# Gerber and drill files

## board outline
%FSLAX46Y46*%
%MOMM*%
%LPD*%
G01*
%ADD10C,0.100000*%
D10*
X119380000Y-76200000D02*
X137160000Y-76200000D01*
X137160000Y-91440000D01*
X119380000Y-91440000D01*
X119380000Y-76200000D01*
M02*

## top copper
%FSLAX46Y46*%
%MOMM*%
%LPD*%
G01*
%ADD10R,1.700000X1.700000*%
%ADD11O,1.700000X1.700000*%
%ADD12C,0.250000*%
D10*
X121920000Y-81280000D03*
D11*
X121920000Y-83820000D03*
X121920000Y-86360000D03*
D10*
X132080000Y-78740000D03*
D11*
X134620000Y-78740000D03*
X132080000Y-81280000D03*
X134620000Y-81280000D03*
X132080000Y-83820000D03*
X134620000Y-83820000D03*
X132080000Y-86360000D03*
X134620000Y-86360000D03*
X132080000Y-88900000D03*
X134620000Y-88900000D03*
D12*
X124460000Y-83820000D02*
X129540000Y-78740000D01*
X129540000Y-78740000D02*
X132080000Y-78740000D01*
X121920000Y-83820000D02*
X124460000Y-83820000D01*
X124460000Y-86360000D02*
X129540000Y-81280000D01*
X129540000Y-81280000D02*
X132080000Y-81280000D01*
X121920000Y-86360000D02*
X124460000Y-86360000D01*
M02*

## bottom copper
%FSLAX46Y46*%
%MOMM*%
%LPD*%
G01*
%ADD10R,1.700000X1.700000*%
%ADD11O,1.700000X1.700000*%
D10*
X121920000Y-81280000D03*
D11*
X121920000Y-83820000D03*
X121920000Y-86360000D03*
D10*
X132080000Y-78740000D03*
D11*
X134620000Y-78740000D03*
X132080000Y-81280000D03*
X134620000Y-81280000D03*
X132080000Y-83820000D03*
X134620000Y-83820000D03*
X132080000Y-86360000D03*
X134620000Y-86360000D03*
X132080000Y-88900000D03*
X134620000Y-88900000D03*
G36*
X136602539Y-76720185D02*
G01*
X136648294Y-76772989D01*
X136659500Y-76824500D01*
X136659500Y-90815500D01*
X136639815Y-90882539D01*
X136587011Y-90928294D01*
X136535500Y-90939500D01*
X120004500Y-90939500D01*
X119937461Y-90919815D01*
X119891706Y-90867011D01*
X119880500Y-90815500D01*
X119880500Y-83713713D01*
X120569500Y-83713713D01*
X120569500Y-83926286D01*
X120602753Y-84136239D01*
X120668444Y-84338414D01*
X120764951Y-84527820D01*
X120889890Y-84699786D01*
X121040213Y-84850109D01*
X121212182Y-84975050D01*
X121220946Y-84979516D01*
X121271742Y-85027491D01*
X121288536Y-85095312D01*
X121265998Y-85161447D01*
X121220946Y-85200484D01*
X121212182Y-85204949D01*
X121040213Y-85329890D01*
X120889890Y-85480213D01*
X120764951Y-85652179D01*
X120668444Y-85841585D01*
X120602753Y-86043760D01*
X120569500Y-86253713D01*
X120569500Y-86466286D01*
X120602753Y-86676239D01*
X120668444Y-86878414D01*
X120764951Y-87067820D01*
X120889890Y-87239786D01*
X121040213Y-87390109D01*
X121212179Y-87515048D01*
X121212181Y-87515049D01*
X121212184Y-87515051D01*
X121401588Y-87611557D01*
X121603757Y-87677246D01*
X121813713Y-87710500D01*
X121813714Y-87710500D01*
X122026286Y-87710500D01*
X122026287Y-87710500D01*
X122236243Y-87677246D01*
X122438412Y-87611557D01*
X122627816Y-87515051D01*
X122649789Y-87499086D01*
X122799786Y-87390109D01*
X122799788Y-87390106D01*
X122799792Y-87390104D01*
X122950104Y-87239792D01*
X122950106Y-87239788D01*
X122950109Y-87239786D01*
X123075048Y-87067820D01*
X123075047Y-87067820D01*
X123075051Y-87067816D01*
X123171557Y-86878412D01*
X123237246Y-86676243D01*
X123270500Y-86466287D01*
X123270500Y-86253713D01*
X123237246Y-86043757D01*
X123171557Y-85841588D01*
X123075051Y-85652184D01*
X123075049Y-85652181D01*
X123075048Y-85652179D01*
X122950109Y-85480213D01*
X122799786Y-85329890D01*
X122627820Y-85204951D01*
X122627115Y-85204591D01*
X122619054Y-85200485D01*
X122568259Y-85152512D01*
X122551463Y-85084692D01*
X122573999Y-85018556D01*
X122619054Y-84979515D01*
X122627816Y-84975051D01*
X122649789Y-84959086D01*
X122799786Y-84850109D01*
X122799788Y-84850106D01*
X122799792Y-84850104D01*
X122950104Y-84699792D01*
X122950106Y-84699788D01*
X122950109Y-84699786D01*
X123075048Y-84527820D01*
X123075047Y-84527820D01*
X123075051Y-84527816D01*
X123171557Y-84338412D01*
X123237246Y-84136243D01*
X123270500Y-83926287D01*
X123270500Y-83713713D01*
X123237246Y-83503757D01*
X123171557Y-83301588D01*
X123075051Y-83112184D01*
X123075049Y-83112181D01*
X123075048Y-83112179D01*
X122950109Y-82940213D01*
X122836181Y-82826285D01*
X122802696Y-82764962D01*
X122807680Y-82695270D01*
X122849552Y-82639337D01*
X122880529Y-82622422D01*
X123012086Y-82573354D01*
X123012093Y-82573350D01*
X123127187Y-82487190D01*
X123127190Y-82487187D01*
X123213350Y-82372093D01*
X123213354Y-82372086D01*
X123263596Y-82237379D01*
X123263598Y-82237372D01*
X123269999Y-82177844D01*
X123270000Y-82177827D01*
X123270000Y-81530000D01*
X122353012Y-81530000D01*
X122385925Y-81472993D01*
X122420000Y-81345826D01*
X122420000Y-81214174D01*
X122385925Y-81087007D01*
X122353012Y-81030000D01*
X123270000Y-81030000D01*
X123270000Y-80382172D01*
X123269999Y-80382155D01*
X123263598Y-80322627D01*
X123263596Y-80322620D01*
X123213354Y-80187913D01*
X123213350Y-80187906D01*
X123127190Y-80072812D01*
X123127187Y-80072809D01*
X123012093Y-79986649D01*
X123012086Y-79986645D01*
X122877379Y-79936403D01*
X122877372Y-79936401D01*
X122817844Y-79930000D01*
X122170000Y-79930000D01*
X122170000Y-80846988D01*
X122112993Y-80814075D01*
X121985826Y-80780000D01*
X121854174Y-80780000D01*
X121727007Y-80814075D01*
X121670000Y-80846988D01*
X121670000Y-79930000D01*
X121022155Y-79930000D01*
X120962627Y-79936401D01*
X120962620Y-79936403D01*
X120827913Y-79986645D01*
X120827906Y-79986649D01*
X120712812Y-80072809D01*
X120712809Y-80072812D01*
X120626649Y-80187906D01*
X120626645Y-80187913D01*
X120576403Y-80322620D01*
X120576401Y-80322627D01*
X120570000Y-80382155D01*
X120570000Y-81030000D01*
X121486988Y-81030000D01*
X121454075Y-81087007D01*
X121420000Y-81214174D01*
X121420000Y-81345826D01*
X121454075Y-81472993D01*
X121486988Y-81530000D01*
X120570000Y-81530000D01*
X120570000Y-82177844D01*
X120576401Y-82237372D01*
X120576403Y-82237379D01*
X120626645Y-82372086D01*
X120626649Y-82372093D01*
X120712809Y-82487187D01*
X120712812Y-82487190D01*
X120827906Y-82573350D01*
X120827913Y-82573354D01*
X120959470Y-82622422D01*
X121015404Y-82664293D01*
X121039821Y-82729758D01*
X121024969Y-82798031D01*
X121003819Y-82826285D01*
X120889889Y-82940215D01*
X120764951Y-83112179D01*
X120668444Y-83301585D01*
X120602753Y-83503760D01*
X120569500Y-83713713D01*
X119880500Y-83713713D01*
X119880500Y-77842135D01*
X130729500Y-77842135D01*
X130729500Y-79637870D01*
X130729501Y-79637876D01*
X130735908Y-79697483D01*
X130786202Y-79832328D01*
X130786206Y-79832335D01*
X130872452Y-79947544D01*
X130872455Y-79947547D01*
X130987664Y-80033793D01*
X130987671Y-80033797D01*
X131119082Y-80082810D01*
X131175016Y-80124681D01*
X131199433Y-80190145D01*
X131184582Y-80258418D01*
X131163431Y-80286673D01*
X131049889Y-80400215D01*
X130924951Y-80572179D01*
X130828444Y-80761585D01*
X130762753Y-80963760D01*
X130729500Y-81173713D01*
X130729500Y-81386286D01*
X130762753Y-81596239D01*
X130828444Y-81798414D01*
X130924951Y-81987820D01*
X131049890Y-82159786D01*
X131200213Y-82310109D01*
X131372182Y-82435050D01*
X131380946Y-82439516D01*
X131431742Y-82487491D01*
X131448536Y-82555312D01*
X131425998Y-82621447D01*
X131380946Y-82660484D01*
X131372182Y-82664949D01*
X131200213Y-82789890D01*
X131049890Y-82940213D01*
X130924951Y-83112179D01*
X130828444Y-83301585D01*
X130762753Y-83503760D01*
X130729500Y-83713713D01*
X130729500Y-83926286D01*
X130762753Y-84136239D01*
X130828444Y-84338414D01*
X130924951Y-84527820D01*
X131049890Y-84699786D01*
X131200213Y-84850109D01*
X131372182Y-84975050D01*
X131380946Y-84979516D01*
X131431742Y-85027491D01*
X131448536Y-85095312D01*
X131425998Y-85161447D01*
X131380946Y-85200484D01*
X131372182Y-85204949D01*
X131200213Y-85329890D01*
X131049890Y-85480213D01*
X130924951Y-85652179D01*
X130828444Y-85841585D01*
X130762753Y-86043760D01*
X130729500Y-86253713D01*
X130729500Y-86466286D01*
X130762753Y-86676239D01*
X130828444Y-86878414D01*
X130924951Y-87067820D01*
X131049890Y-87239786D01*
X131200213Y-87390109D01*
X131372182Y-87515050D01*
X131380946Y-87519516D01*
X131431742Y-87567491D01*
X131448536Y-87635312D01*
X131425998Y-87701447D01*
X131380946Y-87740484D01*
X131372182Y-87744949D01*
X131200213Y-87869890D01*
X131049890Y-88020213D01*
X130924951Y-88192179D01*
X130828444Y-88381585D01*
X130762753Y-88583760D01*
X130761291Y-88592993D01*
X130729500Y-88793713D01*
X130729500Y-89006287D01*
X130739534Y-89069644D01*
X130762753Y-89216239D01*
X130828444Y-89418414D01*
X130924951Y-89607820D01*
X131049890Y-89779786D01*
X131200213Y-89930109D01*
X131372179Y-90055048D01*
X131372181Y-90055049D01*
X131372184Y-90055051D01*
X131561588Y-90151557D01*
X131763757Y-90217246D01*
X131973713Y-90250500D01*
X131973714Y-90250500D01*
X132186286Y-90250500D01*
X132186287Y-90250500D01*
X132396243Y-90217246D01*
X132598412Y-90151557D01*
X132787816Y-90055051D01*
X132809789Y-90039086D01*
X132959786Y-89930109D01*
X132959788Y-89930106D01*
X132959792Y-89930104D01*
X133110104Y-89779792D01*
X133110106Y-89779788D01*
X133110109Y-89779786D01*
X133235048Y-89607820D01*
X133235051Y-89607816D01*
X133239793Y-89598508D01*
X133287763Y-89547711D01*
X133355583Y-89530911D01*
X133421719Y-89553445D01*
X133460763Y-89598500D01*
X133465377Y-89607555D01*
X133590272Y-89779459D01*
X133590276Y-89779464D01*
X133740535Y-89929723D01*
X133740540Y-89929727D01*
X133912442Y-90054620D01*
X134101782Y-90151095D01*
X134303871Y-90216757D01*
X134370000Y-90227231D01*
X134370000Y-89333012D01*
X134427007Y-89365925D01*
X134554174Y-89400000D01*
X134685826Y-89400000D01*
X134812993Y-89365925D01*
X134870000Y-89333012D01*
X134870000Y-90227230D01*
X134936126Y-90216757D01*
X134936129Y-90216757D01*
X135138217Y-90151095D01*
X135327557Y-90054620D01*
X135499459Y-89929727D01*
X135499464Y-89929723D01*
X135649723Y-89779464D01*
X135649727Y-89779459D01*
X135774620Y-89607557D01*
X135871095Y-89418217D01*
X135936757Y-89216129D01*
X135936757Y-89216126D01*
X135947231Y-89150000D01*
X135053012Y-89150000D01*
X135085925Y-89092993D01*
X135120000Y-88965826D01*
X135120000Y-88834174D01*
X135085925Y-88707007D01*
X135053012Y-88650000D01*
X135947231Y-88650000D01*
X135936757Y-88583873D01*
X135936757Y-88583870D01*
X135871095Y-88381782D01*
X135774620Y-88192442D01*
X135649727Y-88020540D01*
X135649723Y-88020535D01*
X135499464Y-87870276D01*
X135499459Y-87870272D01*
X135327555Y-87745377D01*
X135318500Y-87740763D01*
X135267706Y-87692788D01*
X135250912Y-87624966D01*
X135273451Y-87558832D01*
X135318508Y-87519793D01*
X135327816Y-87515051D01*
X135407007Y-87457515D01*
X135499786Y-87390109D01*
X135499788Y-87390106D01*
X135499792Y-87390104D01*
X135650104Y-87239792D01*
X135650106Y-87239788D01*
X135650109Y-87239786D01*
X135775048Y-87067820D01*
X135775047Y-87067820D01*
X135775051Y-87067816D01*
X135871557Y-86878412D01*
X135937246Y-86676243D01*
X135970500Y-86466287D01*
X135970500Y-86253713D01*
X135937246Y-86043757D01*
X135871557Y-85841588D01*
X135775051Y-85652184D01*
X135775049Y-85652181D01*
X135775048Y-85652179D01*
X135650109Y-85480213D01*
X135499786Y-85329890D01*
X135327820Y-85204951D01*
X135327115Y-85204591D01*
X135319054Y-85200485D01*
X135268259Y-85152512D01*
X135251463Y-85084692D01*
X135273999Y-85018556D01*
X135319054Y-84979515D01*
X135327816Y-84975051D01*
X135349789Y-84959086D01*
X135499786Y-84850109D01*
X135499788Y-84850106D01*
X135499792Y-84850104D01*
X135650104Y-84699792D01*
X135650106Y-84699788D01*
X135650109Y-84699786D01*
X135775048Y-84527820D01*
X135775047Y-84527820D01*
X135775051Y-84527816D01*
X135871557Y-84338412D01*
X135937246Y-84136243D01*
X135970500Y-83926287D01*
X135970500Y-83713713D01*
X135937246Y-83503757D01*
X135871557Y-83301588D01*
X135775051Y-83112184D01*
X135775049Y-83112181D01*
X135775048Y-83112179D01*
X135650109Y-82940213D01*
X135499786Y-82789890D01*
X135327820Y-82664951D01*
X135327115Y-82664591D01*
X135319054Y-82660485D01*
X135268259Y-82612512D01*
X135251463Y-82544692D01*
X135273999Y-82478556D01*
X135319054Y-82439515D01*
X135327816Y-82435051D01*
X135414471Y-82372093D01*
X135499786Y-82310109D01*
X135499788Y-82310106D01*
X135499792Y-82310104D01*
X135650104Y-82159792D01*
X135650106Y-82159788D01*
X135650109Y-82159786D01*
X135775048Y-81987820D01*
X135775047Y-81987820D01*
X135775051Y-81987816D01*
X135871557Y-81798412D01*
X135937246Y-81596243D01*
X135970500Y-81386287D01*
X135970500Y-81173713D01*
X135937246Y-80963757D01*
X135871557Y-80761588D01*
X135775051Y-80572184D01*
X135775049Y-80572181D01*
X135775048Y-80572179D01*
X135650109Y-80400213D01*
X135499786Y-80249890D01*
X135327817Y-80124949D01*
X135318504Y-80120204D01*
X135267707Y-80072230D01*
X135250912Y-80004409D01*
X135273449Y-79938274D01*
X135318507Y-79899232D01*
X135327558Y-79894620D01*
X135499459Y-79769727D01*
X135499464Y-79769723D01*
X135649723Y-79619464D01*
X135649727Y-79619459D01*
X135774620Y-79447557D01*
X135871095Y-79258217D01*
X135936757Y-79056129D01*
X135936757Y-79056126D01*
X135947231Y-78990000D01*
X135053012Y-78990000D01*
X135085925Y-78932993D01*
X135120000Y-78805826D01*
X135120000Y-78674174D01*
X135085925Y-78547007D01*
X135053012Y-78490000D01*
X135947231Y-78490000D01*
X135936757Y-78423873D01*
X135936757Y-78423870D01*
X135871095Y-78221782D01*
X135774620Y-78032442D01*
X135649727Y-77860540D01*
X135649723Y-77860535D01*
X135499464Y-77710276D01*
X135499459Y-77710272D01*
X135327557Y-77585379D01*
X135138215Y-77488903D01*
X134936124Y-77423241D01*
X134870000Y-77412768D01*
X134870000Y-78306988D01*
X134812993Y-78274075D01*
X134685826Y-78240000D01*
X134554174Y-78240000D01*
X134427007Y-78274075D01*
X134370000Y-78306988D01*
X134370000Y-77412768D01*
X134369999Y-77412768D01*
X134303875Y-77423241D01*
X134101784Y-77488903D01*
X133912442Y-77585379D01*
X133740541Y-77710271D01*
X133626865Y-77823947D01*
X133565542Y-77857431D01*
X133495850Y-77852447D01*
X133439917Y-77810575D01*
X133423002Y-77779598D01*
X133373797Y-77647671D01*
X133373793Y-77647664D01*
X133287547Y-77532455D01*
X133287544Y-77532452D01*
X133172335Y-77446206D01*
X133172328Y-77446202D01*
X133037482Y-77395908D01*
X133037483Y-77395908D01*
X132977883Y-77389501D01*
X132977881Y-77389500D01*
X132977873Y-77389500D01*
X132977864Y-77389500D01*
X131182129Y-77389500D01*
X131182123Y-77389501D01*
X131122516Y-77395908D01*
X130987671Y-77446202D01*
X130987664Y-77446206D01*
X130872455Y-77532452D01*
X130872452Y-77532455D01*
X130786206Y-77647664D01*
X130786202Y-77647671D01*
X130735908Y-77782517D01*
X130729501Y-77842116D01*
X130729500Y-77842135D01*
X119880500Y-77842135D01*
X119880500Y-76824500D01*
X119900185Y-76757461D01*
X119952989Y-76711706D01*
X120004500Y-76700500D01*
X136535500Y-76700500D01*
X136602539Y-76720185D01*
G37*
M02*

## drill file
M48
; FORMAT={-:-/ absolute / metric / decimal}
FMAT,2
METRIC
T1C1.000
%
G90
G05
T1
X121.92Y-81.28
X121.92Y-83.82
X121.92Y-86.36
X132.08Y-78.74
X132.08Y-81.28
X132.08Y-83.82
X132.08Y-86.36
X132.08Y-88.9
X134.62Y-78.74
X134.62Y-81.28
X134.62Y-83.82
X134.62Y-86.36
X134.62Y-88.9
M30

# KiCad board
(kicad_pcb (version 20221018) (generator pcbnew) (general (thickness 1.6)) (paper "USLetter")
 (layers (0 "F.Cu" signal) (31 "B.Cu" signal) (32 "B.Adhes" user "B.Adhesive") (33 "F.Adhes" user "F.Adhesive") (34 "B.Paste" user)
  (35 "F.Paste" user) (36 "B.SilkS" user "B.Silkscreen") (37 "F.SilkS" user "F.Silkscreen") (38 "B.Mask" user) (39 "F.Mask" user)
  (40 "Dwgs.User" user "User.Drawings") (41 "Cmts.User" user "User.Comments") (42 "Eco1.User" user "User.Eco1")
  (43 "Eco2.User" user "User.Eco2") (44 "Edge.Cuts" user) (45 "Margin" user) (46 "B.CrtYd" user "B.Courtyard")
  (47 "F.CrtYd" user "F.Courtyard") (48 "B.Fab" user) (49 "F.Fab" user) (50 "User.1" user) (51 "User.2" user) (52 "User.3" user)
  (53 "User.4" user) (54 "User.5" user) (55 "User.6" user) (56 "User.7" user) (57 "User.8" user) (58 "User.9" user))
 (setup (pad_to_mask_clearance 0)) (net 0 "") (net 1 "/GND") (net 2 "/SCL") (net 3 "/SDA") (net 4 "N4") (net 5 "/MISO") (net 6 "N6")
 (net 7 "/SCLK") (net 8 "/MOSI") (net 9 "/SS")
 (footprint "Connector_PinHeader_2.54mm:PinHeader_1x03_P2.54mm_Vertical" (layer "F.Cu") (at 121.92 81.28)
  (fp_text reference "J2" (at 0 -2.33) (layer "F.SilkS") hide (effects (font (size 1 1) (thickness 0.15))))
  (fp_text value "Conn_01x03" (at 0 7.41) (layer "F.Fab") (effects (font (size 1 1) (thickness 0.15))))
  (pad "1" thru_hole rect (at 0 0) (size 1.7 1.7) (drill 1) (layers "*.Cu" "*.Mask") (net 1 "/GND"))
  (pad "2" thru_hole oval (at 0 2.54) (size 1.7 1.7) (drill 1) (layers "*.Cu" "*.Mask") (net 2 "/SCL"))
  (pad "3" thru_hole oval (at 0 5.08) (size 1.7 1.7) (drill 1) (layers "*.Cu" "*.Mask") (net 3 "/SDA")))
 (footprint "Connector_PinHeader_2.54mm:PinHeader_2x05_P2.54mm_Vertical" (layer "F.Cu") (at 132.08 78.74)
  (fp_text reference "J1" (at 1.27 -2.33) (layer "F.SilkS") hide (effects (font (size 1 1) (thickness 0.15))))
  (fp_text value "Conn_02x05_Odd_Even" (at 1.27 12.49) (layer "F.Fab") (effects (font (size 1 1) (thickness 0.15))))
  (pad "1" thru_hole rect (at 0 0) (size 1.7 1.7) (drill 1) (layers "*.Cu" "*.Mask") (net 2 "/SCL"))
  (pad "2" thru_hole oval (at 2.54 0) (size 1.7 1.7) (drill 1) (layers "*.Cu" "*.Mask") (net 1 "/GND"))
  (pad "3" thru_hole oval (at 0 2.54) (size 1.7 1.7) (drill 1) (layers "*.Cu" "*.Mask") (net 3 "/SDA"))
  (pad "4" thru_hole oval (at 2.54 2.54) (size 1.7 1.7) (drill 1) (layers "*.Cu" "*.Mask") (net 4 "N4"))
  (pad "5" thru_hole oval (at 0 5.08) (size 1.7 1.7) (drill 1) (layers "*.Cu" "*.Mask") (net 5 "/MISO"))
  (pad "6" thru_hole oval (at 2.54 5.08) (size 1.7 1.7) (drill 1) (layers "*.Cu" "*.Mask") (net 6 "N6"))
  (pad "7" thru_hole oval (at 0 7.62) (size 1.7 1.7) (drill 1) (layers "*.Cu" "*.Mask") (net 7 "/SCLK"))
  (pad "8" thru_hole oval (at 2.54 7.62) (size 1.7 1.7) (drill 1) (layers "*.Cu" "*.Mask") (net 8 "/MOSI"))
  (pad "9" thru_hole oval (at 0 10.16) (size 1.7 1.7) (drill 1) (layers "*.Cu" "*.Mask") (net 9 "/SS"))
  (pad "10" thru_hole oval (at 2.54 10.16) (size 1.7 1.7) (drill 1) (layers "*.Cu" "*.Mask") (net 1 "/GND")))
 (gr_rect (start 119.38 76.2) (end 137.16 91.44) (stroke (width 0.1) (type default)) (fill none) (layer "Edge.Cuts"))
 (segment (start 124.46 83.82) (end 129.54 78.74) (width 0.25) (layer "F.Cu") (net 2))
 (segment (start 129.54 78.74) (end 132.08 78.74) (width 0.25) (layer "F.Cu") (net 2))
 (segment (start 121.92 83.82) (end 124.46 83.82) (width 0.25) (layer "F.Cu") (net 2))
 (segment (start 124.46 86.36) (end 129.54 81.28) (width 0.25) (layer "F.Cu") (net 3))
 (segment (start 129.54 81.28) (end 132.08 81.28) (width 0.25) (layer "F.Cu") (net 3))
 (segment (start 121.92 86.36) (end 124.46 86.36) (width 0.25) (layer "F.Cu") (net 3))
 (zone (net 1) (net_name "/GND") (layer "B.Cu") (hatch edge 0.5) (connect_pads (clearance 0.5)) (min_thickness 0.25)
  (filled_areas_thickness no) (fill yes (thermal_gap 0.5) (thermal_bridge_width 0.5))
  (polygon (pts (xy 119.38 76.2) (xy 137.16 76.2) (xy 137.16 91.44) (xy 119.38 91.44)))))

